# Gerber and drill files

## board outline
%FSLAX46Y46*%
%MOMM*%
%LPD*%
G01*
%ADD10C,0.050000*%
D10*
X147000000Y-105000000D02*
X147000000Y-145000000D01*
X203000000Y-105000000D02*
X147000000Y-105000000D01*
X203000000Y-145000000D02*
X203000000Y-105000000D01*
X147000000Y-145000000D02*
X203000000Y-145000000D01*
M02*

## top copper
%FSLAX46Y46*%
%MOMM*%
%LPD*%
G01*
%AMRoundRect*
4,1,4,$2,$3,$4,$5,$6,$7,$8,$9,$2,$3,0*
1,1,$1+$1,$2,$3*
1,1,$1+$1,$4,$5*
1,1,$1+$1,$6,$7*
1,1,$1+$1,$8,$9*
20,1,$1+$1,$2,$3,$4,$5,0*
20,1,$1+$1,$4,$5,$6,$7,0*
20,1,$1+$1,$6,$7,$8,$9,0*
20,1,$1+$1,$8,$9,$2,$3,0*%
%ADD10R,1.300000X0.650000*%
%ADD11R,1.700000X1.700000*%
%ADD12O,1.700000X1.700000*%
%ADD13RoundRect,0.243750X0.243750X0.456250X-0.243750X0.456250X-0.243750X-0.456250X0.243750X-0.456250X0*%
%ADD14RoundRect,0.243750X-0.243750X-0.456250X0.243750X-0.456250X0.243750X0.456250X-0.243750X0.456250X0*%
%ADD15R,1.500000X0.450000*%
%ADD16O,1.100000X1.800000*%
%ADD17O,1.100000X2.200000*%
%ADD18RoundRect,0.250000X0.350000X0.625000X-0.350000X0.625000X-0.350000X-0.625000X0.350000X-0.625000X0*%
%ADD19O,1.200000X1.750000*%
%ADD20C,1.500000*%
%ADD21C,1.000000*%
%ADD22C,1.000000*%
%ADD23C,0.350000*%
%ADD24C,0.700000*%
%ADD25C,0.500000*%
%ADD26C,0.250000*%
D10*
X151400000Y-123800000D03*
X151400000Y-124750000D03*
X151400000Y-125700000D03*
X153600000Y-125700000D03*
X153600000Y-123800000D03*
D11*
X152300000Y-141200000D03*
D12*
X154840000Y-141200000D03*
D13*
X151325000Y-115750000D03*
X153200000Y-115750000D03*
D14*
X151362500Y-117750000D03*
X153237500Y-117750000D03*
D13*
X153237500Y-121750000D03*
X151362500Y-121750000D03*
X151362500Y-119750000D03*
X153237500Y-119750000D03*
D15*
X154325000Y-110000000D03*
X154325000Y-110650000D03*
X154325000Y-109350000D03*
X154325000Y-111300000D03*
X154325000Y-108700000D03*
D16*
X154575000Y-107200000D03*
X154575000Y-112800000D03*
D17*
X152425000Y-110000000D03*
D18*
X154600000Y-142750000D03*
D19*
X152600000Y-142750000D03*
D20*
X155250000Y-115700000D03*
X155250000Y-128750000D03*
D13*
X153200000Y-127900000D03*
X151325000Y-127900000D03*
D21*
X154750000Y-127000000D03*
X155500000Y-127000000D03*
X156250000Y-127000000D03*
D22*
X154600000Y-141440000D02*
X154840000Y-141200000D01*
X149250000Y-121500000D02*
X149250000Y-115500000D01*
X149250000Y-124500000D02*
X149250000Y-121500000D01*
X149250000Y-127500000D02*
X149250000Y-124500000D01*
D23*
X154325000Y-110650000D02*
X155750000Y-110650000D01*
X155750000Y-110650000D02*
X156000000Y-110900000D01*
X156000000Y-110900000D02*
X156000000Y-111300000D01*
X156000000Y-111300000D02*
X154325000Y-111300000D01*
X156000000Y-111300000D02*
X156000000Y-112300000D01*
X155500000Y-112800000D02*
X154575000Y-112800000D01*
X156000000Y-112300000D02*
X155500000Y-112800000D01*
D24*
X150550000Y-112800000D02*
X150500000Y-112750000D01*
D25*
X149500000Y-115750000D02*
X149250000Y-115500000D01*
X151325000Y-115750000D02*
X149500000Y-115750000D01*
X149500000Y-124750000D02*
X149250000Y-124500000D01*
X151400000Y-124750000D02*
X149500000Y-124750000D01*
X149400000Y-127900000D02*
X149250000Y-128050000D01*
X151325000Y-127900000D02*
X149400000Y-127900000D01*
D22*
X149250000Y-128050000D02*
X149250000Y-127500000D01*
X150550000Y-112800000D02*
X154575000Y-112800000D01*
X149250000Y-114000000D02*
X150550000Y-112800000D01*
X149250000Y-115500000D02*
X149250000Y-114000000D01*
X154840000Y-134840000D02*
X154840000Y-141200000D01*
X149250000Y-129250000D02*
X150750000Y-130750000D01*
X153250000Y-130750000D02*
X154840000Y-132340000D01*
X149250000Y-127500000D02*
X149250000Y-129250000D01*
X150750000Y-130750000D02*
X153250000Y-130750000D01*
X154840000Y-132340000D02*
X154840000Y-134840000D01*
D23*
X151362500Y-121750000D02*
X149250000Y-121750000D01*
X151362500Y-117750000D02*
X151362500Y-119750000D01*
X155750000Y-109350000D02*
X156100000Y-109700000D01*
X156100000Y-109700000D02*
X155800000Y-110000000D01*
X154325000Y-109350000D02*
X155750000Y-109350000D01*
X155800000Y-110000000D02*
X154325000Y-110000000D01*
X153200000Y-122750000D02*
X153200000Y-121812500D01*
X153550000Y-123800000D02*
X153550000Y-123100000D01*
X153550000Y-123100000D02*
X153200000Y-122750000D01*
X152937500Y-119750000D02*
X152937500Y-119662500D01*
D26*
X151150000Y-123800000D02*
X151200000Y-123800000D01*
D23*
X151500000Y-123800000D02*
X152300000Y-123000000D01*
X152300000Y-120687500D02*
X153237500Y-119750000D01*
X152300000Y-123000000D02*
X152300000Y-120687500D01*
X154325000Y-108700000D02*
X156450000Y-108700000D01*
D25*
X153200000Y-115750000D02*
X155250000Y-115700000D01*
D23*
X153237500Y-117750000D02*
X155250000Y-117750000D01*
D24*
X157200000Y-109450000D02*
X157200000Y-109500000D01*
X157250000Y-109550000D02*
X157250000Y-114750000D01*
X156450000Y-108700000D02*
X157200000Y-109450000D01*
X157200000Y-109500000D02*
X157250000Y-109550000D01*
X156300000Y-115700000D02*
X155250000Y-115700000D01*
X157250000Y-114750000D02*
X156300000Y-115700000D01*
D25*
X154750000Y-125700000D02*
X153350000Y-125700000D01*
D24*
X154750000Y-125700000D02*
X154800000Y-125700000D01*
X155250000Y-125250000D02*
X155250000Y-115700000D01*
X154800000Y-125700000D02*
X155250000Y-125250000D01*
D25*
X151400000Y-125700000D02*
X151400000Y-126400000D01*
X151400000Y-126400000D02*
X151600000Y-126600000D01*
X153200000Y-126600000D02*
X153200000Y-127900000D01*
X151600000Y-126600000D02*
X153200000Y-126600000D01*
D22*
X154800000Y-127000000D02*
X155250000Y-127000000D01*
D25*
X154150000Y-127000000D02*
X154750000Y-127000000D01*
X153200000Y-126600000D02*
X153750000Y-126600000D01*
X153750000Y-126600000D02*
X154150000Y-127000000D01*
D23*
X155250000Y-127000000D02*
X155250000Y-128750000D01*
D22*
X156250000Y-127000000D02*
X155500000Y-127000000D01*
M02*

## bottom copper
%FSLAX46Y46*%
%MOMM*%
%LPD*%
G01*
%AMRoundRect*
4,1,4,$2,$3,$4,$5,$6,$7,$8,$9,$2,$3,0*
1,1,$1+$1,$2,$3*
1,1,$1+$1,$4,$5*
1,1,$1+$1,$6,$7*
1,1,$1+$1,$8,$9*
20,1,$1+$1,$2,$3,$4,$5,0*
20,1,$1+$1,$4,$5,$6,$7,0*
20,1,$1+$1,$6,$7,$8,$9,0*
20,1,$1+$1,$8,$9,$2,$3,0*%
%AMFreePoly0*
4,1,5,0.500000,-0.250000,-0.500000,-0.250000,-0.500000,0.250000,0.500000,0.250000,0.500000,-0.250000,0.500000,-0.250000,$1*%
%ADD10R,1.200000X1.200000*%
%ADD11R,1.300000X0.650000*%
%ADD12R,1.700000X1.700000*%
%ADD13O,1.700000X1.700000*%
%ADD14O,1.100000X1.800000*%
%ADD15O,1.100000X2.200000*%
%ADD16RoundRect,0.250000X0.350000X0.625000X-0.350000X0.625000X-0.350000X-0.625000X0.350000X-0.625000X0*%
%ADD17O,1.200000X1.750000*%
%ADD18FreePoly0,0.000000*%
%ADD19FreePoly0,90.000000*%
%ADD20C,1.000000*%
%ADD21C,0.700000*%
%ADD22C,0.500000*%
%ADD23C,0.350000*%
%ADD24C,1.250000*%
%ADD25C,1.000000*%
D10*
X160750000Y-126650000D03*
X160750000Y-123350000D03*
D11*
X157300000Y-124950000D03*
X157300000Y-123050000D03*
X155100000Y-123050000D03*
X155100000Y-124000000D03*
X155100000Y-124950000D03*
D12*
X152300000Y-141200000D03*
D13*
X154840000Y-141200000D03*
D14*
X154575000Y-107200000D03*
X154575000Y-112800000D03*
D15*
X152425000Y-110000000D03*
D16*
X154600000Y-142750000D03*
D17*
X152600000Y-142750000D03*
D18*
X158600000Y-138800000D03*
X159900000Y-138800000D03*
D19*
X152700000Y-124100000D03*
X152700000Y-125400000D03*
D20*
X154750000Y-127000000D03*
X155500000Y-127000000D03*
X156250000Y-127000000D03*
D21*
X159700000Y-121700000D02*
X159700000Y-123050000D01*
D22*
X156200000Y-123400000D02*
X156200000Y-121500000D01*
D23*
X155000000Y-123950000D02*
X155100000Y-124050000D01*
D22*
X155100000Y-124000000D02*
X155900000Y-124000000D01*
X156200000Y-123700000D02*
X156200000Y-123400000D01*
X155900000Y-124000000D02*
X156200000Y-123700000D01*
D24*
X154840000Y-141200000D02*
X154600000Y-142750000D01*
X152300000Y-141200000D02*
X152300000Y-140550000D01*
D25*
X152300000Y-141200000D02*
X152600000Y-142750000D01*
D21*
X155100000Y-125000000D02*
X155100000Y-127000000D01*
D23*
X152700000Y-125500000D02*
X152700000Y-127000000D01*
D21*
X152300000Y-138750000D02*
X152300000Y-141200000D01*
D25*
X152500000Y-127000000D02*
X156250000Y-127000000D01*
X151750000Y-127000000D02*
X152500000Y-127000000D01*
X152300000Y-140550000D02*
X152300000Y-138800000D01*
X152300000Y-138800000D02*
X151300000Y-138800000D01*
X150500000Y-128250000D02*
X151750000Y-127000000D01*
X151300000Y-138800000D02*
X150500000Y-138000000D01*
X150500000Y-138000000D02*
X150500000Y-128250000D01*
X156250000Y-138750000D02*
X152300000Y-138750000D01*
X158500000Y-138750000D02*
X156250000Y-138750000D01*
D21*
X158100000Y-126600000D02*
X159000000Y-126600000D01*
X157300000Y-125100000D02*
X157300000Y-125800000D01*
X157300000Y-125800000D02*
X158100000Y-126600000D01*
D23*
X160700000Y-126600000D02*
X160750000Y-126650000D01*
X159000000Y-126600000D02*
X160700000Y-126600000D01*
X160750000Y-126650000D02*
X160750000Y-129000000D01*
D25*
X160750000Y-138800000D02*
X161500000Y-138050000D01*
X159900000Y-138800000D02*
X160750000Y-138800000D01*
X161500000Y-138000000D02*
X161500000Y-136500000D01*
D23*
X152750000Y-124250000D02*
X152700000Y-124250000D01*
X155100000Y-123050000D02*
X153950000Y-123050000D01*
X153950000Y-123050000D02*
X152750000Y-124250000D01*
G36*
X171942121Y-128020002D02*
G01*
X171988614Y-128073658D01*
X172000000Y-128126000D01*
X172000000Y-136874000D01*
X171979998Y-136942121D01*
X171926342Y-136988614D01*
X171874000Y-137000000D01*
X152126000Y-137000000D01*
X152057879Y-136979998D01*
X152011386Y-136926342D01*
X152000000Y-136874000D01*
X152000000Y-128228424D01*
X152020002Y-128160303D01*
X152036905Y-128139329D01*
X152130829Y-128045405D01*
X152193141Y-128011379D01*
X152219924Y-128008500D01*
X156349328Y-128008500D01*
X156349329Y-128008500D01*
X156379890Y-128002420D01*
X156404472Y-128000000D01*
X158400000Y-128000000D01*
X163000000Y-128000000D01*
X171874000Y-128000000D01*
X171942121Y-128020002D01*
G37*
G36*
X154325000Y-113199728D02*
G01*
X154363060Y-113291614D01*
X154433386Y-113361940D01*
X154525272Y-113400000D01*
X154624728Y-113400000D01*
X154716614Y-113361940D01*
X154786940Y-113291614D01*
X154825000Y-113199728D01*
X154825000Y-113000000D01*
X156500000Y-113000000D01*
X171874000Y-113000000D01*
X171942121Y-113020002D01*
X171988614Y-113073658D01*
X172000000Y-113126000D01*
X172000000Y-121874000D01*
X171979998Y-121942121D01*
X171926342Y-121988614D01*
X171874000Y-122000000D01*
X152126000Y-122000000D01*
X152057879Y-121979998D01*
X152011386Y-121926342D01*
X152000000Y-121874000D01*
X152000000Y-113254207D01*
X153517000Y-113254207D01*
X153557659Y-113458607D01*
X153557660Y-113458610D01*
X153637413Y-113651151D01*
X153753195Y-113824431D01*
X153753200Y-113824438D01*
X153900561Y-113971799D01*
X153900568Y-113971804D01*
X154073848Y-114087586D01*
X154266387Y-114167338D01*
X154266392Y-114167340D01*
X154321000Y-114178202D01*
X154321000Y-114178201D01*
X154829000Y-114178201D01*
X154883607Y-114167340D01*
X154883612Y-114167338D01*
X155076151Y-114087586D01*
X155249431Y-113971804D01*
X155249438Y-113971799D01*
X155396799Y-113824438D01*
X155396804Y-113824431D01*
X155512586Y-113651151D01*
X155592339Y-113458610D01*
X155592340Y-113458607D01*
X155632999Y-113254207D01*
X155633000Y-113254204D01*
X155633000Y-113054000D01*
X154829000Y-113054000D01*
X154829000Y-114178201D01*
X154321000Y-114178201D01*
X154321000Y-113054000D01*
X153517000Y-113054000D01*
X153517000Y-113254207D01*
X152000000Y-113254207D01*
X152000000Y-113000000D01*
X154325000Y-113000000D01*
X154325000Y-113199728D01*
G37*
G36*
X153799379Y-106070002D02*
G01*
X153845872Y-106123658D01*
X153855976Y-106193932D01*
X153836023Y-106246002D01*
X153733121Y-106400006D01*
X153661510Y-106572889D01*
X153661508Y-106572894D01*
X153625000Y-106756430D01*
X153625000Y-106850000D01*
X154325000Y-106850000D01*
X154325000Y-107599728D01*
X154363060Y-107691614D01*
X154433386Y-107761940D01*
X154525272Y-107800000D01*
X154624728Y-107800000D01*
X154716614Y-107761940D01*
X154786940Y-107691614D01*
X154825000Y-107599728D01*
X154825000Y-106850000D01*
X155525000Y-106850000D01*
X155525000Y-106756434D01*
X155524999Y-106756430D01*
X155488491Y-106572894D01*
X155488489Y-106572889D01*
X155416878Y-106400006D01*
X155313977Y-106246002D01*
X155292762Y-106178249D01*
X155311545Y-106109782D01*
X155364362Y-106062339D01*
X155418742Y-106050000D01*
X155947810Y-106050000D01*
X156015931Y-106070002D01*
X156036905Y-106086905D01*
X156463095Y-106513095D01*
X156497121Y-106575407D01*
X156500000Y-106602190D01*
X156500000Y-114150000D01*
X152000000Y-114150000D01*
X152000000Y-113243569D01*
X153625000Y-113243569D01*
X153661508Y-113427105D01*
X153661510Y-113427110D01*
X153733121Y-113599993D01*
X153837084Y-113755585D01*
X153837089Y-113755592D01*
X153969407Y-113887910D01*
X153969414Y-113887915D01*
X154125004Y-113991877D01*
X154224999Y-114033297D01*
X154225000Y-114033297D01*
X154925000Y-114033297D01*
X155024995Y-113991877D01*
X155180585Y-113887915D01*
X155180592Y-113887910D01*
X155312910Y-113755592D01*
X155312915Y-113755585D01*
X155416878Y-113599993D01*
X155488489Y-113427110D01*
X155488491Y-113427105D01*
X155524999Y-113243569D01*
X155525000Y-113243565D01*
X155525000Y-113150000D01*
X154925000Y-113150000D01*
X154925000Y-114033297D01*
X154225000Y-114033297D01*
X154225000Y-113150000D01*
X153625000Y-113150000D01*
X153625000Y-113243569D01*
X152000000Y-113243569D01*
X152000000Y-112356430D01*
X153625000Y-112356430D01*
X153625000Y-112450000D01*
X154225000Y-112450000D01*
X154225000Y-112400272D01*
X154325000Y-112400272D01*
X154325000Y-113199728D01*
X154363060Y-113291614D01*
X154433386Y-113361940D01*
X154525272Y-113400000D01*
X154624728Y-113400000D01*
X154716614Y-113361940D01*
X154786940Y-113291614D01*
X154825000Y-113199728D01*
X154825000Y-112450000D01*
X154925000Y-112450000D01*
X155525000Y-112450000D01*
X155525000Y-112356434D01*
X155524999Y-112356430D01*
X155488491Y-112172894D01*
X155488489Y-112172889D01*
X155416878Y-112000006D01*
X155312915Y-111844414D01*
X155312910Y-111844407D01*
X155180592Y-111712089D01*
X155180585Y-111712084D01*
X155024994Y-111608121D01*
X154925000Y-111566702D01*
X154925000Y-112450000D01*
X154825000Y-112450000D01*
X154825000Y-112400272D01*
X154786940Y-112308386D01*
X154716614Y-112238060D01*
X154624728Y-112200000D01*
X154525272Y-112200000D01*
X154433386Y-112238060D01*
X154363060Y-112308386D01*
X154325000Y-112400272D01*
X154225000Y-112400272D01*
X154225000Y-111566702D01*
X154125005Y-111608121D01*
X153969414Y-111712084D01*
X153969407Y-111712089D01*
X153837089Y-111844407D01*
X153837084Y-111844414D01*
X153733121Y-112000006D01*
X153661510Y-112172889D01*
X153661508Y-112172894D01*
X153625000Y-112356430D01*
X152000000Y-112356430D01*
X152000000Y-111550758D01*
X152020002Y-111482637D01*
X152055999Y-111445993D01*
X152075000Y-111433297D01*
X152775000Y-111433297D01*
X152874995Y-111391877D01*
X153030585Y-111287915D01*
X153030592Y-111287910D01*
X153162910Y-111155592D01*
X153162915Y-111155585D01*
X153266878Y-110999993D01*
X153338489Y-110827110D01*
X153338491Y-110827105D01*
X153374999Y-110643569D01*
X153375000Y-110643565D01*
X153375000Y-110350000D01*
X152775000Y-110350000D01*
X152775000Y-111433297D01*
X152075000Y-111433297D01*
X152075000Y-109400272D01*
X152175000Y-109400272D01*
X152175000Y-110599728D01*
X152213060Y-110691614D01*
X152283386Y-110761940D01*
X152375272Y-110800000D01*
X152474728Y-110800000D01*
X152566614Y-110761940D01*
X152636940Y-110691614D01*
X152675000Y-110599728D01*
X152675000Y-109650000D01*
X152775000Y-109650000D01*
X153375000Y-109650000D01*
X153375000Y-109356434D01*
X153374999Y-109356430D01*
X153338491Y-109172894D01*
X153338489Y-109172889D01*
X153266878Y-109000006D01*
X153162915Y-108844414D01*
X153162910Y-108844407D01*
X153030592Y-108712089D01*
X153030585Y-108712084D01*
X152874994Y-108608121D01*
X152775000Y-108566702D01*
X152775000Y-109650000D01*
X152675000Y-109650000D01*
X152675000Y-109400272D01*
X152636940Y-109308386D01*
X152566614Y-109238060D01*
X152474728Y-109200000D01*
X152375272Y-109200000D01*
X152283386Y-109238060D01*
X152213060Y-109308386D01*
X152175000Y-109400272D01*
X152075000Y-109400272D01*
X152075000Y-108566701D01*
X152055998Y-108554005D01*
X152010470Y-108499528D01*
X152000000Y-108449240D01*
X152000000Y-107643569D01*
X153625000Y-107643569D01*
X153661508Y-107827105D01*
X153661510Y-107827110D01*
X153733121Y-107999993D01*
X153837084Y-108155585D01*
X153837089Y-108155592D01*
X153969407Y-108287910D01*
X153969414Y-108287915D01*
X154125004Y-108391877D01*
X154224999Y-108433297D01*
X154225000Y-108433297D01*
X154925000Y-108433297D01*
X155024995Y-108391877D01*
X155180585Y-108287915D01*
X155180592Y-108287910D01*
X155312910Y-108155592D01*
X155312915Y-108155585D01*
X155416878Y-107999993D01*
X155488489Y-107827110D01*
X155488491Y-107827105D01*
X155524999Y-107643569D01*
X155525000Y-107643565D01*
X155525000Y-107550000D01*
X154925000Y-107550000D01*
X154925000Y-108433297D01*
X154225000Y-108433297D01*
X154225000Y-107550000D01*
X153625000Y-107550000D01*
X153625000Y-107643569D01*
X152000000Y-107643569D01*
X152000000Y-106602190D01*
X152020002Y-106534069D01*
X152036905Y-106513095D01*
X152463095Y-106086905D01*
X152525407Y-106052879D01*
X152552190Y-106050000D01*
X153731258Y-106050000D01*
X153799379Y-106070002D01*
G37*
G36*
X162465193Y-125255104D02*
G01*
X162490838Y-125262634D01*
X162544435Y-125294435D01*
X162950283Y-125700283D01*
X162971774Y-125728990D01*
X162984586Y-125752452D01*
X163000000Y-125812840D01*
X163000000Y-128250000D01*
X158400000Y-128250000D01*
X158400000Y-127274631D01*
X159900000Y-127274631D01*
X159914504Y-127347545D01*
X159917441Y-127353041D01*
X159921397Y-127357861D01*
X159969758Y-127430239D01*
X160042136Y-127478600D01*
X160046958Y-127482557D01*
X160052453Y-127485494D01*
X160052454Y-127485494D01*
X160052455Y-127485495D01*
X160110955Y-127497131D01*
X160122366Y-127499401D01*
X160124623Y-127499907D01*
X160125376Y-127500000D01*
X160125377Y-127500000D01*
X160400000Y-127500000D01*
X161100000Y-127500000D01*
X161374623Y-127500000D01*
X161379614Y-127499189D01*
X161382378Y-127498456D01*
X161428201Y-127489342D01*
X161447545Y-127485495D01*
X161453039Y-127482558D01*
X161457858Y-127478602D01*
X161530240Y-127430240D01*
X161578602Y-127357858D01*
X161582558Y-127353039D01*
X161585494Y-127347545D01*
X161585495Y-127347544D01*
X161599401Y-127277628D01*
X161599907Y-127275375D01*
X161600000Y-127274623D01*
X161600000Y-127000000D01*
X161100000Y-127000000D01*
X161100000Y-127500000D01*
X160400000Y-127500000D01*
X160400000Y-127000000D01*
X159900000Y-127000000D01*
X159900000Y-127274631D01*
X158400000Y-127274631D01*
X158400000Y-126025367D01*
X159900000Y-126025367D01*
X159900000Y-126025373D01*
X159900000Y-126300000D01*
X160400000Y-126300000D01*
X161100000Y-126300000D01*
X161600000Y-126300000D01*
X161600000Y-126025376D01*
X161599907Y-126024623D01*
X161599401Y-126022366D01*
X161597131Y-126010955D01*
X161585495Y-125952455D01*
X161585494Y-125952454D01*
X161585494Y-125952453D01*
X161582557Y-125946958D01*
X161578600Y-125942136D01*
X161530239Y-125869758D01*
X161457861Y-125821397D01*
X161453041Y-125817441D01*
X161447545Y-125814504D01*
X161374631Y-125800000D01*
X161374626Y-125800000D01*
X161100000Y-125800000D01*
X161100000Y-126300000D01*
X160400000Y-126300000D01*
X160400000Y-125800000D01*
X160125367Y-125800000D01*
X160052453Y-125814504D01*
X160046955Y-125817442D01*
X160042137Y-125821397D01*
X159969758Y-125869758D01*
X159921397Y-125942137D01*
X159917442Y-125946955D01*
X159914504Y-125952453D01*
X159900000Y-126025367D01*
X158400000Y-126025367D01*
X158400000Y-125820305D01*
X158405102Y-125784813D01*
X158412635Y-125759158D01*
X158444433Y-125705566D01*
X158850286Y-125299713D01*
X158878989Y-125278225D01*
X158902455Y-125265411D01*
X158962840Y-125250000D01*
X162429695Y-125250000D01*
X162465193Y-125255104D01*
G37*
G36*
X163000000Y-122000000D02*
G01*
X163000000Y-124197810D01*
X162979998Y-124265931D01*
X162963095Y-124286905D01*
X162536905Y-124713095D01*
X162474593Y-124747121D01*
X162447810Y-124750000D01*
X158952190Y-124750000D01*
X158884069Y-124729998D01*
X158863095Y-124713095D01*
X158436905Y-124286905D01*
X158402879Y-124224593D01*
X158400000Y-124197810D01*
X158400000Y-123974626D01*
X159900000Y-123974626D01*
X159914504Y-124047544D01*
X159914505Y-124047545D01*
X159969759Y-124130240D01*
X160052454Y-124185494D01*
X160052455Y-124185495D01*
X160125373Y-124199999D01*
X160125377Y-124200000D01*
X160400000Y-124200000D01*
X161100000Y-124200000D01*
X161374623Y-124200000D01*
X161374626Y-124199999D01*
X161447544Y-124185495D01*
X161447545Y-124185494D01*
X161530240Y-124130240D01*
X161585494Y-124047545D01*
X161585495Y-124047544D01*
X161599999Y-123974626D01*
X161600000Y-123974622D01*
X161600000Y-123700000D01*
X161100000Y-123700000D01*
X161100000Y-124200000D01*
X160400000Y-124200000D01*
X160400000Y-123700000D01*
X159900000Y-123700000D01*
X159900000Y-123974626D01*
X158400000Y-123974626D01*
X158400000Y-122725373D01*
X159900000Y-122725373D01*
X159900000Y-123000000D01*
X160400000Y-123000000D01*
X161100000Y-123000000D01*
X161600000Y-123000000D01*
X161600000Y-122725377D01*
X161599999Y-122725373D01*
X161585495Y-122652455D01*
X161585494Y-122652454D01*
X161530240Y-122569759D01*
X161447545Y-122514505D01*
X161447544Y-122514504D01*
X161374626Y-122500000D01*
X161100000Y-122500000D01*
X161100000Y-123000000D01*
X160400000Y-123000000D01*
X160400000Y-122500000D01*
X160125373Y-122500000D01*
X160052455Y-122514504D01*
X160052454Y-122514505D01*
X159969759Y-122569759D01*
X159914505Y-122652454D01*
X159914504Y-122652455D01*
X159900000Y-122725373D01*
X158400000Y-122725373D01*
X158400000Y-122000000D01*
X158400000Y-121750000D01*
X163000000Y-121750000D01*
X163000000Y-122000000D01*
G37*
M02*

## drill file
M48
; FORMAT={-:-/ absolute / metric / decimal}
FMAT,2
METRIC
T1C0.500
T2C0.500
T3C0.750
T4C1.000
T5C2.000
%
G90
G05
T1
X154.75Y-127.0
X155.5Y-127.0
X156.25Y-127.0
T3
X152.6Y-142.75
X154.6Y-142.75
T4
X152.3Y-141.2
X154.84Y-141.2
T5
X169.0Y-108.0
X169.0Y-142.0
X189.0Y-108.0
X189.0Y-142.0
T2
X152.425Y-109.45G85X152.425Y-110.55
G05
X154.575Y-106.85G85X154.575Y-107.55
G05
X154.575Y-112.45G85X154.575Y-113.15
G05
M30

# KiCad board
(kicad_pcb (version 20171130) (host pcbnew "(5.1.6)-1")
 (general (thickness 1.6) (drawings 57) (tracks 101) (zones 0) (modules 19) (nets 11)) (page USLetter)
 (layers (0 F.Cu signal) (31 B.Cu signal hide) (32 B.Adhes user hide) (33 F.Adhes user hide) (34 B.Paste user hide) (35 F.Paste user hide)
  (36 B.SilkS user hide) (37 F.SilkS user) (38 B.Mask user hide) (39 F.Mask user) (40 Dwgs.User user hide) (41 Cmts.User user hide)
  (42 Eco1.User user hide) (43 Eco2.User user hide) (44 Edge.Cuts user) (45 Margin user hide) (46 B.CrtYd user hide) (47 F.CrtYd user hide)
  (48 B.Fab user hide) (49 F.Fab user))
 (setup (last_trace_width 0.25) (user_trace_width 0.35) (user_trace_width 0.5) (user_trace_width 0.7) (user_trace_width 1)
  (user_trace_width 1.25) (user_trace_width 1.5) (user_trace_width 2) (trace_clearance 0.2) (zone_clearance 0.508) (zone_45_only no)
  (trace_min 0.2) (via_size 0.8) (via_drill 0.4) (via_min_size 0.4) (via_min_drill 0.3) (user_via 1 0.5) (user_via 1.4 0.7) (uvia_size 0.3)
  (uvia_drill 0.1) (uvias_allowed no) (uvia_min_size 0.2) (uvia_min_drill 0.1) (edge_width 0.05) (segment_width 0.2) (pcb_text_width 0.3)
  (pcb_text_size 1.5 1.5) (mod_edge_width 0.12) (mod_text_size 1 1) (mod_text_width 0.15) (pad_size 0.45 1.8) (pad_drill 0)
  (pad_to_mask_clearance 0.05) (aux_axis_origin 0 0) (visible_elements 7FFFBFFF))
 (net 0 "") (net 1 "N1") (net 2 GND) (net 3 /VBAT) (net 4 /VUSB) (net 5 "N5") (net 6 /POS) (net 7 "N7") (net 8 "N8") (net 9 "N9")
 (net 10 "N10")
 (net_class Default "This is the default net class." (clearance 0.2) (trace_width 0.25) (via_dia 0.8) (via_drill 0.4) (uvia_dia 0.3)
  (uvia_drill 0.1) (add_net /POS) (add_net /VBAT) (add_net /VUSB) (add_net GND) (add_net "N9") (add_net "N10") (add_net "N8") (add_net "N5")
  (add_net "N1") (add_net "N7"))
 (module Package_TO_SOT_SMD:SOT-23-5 (layer F.Cu) (at 152.5 124.75)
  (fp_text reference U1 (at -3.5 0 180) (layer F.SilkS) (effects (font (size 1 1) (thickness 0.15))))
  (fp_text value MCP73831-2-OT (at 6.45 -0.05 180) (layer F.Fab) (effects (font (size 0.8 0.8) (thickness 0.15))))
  (pad 1 smd rect (at -1.1 -0.95) (size 1.3 0.65) (layers F.Cu F.Paste F.Mask) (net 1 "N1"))
  (pad 2 smd rect (at -1.1 0) (size 1.3 0.65) (layers F.Cu F.Paste F.Mask) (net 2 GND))
  (pad 3 smd rect (at -1.1 0.95) (size 1.3 0.65) (layers F.Cu F.Paste F.Mask) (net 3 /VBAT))
  (pad 4 smd rect (at 1.1 0.95) (size 1.3 0.65) (layers F.Cu F.Paste F.Mask) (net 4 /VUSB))
  (pad 5 smd rect (at 1.1 -0.95) (size 1.3 0.65) (layers F.Cu F.Paste F.Mask) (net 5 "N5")))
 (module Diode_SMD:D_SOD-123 (layer B.Cu) (at 160.75 125 90)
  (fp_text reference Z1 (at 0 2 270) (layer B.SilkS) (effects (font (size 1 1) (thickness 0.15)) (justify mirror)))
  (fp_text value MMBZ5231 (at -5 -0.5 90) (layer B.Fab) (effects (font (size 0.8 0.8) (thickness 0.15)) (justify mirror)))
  (pad 1 smd rect (at -1.65 0 90) (size 1.2 1.2) (layers B.Cu B.Paste B.Mask) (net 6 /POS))
  (pad 2 smd rect (at 1.65 0 90) (size 1.2 1.2) (layers B.Cu B.Paste B.Mask) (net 2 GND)))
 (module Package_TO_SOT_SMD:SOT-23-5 (layer B.Cu) (at 156.2 124)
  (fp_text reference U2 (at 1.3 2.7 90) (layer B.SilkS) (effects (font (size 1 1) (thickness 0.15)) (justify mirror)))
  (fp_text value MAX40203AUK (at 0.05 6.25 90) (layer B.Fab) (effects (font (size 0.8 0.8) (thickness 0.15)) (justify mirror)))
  (pad 5 smd rect (at 1.1 0.95) (size 1.3 0.65) (layers B.Cu B.Paste B.Mask) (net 6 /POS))
  (pad 4 smd rect (at 1.1 -0.95) (size 1.3 0.65) (layers B.Cu B.Paste B.Mask) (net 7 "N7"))
  (pad 3 smd rect (at -1.1 -0.95) (size 1.3 0.65) (layers B.Cu B.Paste B.Mask) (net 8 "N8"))
  (pad 2 smd rect (at -1.1 0) (size 1.3 0.65) (layers B.Cu B.Paste B.Mask) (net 2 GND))
  (pad 1 smd rect (at -1.1 0.95) (size 1.3 0.65) (layers B.Cu B.Paste B.Mask) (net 3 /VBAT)))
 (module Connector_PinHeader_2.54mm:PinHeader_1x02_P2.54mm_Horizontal (layer F.Cu) (at 152.3 141.2 90)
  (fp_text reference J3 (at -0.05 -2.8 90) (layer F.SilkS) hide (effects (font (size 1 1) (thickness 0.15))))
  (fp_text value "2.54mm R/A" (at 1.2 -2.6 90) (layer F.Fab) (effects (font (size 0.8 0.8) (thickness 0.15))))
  (pad 1 thru_hole rect (at 0 0 90) (size 1.7 1.7) (drill 1) (layers *.Cu *.Mask) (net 3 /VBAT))
  (pad 2 thru_hole oval (at 0 2.54 90) (size 1.7 1.7) (drill 1) (layers *.Cu *.Mask) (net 2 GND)))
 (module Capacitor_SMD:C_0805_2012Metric (layer F.Cu) (at 152.2625 115.75 180)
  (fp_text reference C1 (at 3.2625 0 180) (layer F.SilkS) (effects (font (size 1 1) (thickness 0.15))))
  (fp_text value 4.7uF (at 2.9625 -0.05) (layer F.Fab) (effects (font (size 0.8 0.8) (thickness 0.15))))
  (pad 2 smd roundrect (at 0.9375 0 180) (size 0.975 1.4) (layers F.Cu F.Paste F.Mask) (roundrect_rratio 0.25) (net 2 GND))
  (pad 1 smd roundrect (at -0.9375 0 180) (size 0.975 1.4) (layers F.Cu F.Paste F.Mask) (roundrect_rratio 0.25) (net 4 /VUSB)))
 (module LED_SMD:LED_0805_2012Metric (layer F.Cu) (at 152.3 117.75)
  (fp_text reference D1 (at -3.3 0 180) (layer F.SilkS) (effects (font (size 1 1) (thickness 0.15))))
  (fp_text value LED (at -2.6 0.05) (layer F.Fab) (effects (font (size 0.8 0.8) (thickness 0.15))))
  (pad 1 smd roundrect (at -0.9375 0) (size 0.975 1.4) (layers F.Cu F.Paste F.Mask) (roundrect_rratio 0.25) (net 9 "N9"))
  (pad 2 smd roundrect (at 0.9375 0) (size 0.975 1.4) (layers F.Cu F.Paste F.Mask) (roundrect_rratio 0.25) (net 4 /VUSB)))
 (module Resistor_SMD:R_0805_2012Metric (layer F.Cu) (at 152.3 121.75 180)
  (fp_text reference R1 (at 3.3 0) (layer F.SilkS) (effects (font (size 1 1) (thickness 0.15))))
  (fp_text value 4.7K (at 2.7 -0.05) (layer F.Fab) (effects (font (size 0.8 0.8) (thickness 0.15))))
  (pad 1 smd roundrect (at -0.9375 0 180) (size 0.975 1.4) (layers F.Cu F.Paste F.Mask) (roundrect_rratio 0.25) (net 5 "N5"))
  (pad 2 smd roundrect (at 0.9375 0 180) (size 0.975 1.4) (layers F.Cu F.Paste F.Mask) (roundrect_rratio 0.25) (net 2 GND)))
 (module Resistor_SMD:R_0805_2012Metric (layer F.Cu) (at 152.3 119.75 180)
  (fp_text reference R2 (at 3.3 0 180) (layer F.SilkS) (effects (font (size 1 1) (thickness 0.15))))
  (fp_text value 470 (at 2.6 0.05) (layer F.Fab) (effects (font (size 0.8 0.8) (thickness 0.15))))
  (pad 2 smd roundrect (at 0.9375 0 180) (size 0.975 1.4) (layers F.Cu F.Paste F.Mask) (roundrect_rratio 0.25) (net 9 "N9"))
  (pad 1 smd roundrect (at -0.9375 0 180) (size 0.975 1.4) (layers F.Cu F.Paste F.Mask) (roundrect_rratio 0.25) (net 1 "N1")))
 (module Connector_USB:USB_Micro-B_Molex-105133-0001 (layer F.Cu) (at 153.5 110 270)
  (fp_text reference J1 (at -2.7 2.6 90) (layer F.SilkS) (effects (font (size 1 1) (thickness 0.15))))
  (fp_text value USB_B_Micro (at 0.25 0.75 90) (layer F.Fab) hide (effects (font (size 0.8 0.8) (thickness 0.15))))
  (pad 3 smd rect (at 0 -0.825 270) (size 0.45 1.5) (layers F.Cu F.Paste F.Mask) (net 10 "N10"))
  (pad 4 smd rect (at 0.65 -0.825 270) (size 0.45 1.5) (layers F.Cu F.Paste F.Mask) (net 2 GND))
  (pad 2 smd rect (at -0.65 -0.825 270) (size 0.45 1.5) (layers F.Cu F.Paste F.Mask) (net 10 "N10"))
  (pad 5 smd rect (at 1.3 -0.825 270) (size 0.45 1.5) (layers F.Cu F.Paste F.Mask) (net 2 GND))
  (pad 1 smd rect (at -1.3 -0.825 270) (size 0.45 1.5) (layers F.Cu F.Paste F.Mask) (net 4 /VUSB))
  (pad 6 thru_hole oval (at -2.8 -1.075 270) (size 1.8 1.1) (drill oval 1.2 0.5) (layers *.Cu *.Mask) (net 2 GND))
  (pad 6 thru_hole oval (at 2.8 -1.075 270) (size 1.8 1.1) (drill oval 1.2 0.5) (layers *.Cu *.Mask) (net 2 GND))
  (pad 6 thru_hole oval (at 0 1.075 270) (size 2.2 1.1) (drill oval 1.6 0.5) (layers *.Cu *.Mask) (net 2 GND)))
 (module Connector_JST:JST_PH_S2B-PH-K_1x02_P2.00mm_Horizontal (layer F.Cu) (at 154.6 142.75 180)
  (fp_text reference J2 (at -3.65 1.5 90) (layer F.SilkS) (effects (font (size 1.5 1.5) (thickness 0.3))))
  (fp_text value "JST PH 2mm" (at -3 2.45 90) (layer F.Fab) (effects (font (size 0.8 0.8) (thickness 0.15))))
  (pad 1 thru_hole roundrect (at 0 0 180) (size 1.2 1.75) (drill 0.75) (layers *.Cu *.Mask) (roundrect_rratio 0.208333) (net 2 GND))
  (pad 2 thru_hole oval (at 2 0 180) (size 1.2 1.75) (drill 0.75) (layers *.Cu *.Mask) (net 3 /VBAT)))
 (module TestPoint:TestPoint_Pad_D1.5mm (layer F.Cu) (at 155.25 115.7 270)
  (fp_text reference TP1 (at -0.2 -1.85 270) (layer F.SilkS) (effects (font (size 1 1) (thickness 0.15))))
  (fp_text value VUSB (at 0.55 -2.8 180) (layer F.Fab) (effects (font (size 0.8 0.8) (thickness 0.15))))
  (pad 1 smd circle (at 0 0 270) (size 1.5 1.5) (layers F.Cu F.Mask) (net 4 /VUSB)))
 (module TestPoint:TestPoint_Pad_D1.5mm (layer F.Cu) (at 155.25 128.75)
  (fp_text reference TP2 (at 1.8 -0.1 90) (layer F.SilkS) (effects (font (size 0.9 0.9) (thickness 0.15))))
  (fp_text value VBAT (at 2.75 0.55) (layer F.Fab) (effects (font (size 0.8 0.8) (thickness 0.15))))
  (pad 1 smd circle (at 0 0) (size 1.5 1.5) (layers F.Cu F.Mask) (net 3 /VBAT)))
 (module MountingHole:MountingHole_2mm (layer F.Cu) (at 189 108)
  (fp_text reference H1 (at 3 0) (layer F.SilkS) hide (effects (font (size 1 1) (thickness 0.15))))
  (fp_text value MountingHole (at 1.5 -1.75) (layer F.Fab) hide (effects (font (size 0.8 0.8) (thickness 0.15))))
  (pad "" np_thru_hole circle (at 0 0) (size 2 2) (drill 2) (layers *.Cu *.Mask)))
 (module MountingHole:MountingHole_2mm (layer F.Cu) (at 169 108)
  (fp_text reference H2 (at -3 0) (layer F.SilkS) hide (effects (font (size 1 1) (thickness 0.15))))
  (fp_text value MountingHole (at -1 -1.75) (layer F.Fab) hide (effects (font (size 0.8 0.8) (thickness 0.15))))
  (pad "" np_thru_hole circle (at 0 0) (size 2 2) (drill 2) (layers *.Cu *.Mask)))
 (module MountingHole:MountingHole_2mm (layer F.Cu) (at 189 142)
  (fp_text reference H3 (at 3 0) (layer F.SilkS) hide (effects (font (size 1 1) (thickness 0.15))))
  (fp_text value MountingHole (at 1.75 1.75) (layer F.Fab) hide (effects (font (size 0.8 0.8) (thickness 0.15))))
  (pad "" np_thru_hole circle (at 0 0) (size 2 2) (drill 2) (layers *.Cu *.Mask)))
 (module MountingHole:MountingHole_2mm (layer F.Cu) (at 169 142)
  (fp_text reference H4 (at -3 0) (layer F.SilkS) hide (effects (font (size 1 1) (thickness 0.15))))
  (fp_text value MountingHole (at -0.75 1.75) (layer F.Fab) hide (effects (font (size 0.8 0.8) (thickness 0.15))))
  (pad "" np_thru_hole circle (at 0 0) (size 2 2) (drill 2) (layers *.Cu *.Mask)))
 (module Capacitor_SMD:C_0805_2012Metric (layer F.Cu) (at 152.2625 127.9 180)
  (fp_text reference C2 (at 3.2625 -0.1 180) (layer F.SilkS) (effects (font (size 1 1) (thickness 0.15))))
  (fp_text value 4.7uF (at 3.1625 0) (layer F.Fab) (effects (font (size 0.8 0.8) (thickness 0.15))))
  (pad 1 smd roundrect (at -0.9375 0 180) (size 0.975 1.4) (layers F.Cu F.Paste F.Mask) (roundrect_rratio 0.25) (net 3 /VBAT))
  (pad 2 smd roundrect (at 0.9375 0 180) (size 0.975 1.4) (layers F.Cu F.Paste F.Mask) (roundrect_rratio 0.25) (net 2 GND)))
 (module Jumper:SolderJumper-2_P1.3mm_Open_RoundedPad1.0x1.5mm (layer B.Cu) (at 159.25 138.8)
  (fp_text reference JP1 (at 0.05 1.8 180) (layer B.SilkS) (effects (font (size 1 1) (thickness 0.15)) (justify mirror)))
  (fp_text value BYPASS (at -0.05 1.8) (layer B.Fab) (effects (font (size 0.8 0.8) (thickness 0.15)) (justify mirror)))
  (pad 1 smd custom (at -0.65 0) (size 1 0.5) (layers B.Cu B.Mask) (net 3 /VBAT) (zone_connect 2)
   (options (clearance outline) (anchor rect)) (primitives))
  (pad 2 smd custom (at 0.65 0) (size 1 0.5) (layers B.Cu B.Mask) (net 6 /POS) (zone_connect 2) (options (clearance outline) (anchor rect))
   (primitives)))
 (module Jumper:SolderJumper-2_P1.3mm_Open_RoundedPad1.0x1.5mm (layer B.Cu) (at 152.7 124.75 90)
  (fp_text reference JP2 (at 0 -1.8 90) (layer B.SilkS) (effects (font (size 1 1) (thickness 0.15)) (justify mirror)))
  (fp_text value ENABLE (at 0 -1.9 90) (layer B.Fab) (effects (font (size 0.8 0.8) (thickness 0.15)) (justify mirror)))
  (pad 2 smd custom (at 0.65 0 90) (size 1 0.5) (layers B.Cu B.Mask) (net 8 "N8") (zone_connect 2)
   (options (clearance outline) (anchor rect)) (primitives))
  (pad 1 smd custom (at -0.65 0 90) (size 1 0.5) (layers B.Cu B.Mask) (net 3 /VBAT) (zone_connect 2)
   (options (clearance outline) (anchor rect)) (primitives)))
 (gr_line (start 147 105) (end 147 145) (layer Edge.Cuts) (width 0.05))
 (gr_line (start 203 105) (end 147 105) (layer Edge.Cuts) (width 0.05))
 (gr_line (start 203 145) (end 203 105) (layer Edge.Cuts) (width 0.05))
 (gr_line (start 147 145) (end 203 145) (layer Edge.Cuts) (width 0.05))
 (segment (start 159.7 121.7) (end 159.7 123.05) (width 0.7) (layer B.Cu) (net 2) (status 20))
 (segment (start 156.2 123.4) (end 156.2 121.5) (width 0.5) (layer B.Cu) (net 2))
 (segment (start 155 123.95) (end 155.1 124.05) (width 0.35) (layer B.Cu) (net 2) (status 30))
 (segment (start 155.1 124) (end 155.9 124) (width 0.5) (layer B.Cu) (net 2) (status 10))
 (segment (start 156.2 123.7) (end 156.2 123.4) (width 0.5) (layer B.Cu) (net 2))
 (segment (start 155.9 124) (end 156.2 123.7) (width 0.5) (layer B.Cu) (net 2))
 (segment (start 154.6 141.44) (end 154.84 141.2) (width 1) (layer F.Cu) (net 2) (status 30))
 (segment (start 149.25 121.5) (end 149.25 115.5) (width 1) (layer F.Cu) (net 2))
 (segment (start 149.25 124.5) (end 149.25 121.5) (width 1) (layer F.Cu) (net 2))
 (segment (start 149.25 127.5) (end 149.25 124.5) (width 1) (layer F.Cu) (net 2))
 (segment (start 154.325 110.65) (end 155.75 110.65) (width 0.35) (layer F.Cu) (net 2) (status 10))
 (segment (start 155.75 110.65) (end 156 110.9) (width 0.35) (layer F.Cu) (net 2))
 (segment (start 156 110.9) (end 156 111.3) (width 0.35) (layer F.Cu) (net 2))
 (segment (start 156 111.3) (end 154.325 111.3) (width 0.35) (layer F.Cu) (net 2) (status 20))
 (segment (start 156 111.3) (end 156 112.3) (width 0.35) (layer F.Cu) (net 2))
 (segment (start 155.5 112.8) (end 154.575 112.8) (width 0.35) (layer F.Cu) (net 2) (status 20))
 (segment (start 156 112.3) (end 155.5 112.8) (width 0.35) (layer F.Cu) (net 2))
 (segment (start 150.55 112.8) (end 150.5 112.75) (width 0.7) (layer F.Cu) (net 2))
 (segment (start 149.5 115.75) (end 149.25 115.5) (width 0.5) (layer F.Cu) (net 2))
 (segment (start 151.325 115.75) (end 149.5 115.75) (width 0.5) (layer F.Cu) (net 2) (status 10))
 (segment (start 149.5 124.75) (end 149.25 124.5) (width 0.5) (layer F.Cu) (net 2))
 (segment (start 151.4 124.75) (end 149.5 124.75) (width 0.5) (layer F.Cu) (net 2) (status 10))
 (segment (start 149.4 127.9) (end 149.25 128.05) (width 0.5) (layer F.Cu) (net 2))
 (segment (start 151.325 127.9) (end 149.4 127.9) (width 0.5) (layer F.Cu) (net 2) (status 10))
 (segment (start 149.25 128.05) (end 149.25 127.5) (width 1) (layer F.Cu) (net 2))
 (segment (start 154.84 141.2) (end 154.6 142.75) (width 1.25) (layer B.Cu) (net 2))
 (segment (start 150.55 112.8) (end 154.575 112.8) (width 1) (layer F.Cu) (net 2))
 (segment (start 149.25 114) (end 150.55 112.8) (width 1) (layer F.Cu) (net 2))
 (segment (start 149.25 115.5) (end 149.25 114) (width 1) (layer F.Cu) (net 2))
 (segment (start 154.84 134.84) (end 154.84 141.2) (width 1) (layer F.Cu) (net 2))
 (segment (start 149.25 129.25) (end 150.75 130.75) (width 1) (layer F.Cu) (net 2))
 (segment (start 153.25 130.75) (end 154.84 132.34) (width 1) (layer F.Cu) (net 2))
 (segment (start 149.25 127.5) (end 149.25 129.25) (width 1) (layer F.Cu) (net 2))
 (segment (start 150.75 130.75) (end 153.25 130.75) (width 1) (layer F.Cu) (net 2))
 (segment (start 154.84 132.34) (end 154.84 134.84) (width 1) (layer F.Cu) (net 2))
 (segment (start 151.3625 121.75) (end 149.25 121.75) (width 0.35) (layer F.Cu) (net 2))
 (segment (start 151.3625 117.75) (end 151.3625 119.75) (width 0.35) (layer F.Cu) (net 9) (status 30))
 (segment (start 155.75 109.35) (end 156.1 109.7) (width 0.35) (layer F.Cu) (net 10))
 (segment (start 156.1 109.7) (end 155.8 110) (width 0.35) (layer F.Cu) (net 10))
 (segment (start 154.325 109.35) (end 155.75 109.35) (width 0.35) (layer F.Cu) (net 10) (status 10))
 (segment (start 155.8 110) (end 154.325 110) (width 0.35) (layer F.Cu) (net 10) (status 20))
 (segment (start 153.2 122.75) (end 153.2 121.8125) (width 0.35) (layer F.Cu) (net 5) (status 20))
 (segment (start 153.55 123.8) (end 153.55 123.1) (width 0.35) (layer F.Cu) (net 5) (status 10))
 (segment (start 153.55 123.1) (end 153.2 122.75) (width 0.35) (layer F.Cu) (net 5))
 (segment (start 152.9375 119.75) (end 152.9375 119.6625) (width 0.35) (layer F.Cu) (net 1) (status 30))
 (segment (start 151.15 123.8) (end 151.2 123.8) (width 0.25) (layer F.Cu) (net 1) (status 30))
 (segment (start 151.5 123.8) (end 152.3 123) (width 0.35) (layer F.Cu) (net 1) (status 10))
 (segment (start 152.3 120.6875) (end 153.2375 119.75) (width 0.35) (layer F.Cu) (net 1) (status 20))
 (segment (start 152.3 123) (end 152.3 120.6875) (width 0.35) (layer F.Cu) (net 1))
 (segment (start 154.325 108.7) (end 156.45 108.7) (width 0.35) (layer F.Cu) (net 4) (status 10))
 (segment (start 153.2 115.75) (end 155.25 115.7) (width 0.5) (layer F.Cu) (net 4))
 (segment (start 153.2375 117.75) (end 155.25 117.75) (width 0.35) (layer F.Cu) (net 4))
 (segment (start 157.2 109.45) (end 157.2 109.5) (width 0.7) (layer F.Cu) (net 4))
 (segment (start 157.25 109.55) (end 157.25 114.75) (width 0.7) (layer F.Cu) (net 4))
 (segment (start 156.45 108.7) (end 157.2 109.45) (width 0.7) (layer F.Cu) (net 4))
 (segment (start 157.2 109.5) (end 157.25 109.55) (width 0.7) (layer F.Cu) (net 4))
 (segment (start 156.3 115.7) (end 155.25 115.7) (width 0.7) (layer F.Cu) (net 4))
 (segment (start 157.25 114.75) (end 156.3 115.7) (width 0.7) (layer F.Cu) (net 4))
 (segment (start 154.75 125.7) (end 153.35 125.7) (width 0.5) (layer F.Cu) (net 4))
 (segment (start 154.75 125.7) (end 154.8 125.7) (width 0.7) (layer F.Cu) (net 4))
 (segment (start 155.25 125.25) (end 155.25 115.7) (width 0.7) (layer F.Cu) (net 4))
 (segment (start 154.8 125.7) (end 155.25 125.25) (width 0.7) (layer F.Cu) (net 4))
 (segment (start 151.4 125.7) (end 151.4 126.4) (width 0.5) (layer F.Cu) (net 3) (status 10))
 (segment (start 151.4 126.4) (end 151.6 126.6) (width 0.5) (layer F.Cu) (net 3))
 (segment (start 153.2 126.6) (end 153.2 127.9) (width 0.5) (layer F.Cu) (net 3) (status 20))
 (segment (start 151.6 126.6) (end 153.2 126.6) (width 0.5) (layer F.Cu) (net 3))
 (via (at 154.75 127) (size 1) (drill 0.5) (layers F.Cu B.Cu) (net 3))
 (via (at 155.5 127) (size 1) (drill 0.5) (layers F.Cu B.Cu) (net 3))
 (segment (start 152.3 141.2) (end 152.3 140.55) (width 1.25) (layer B.Cu) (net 3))
 (segment (start 152.3 141.2) (end 152.6 142.75) (width 1) (layer B.Cu) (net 3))
 (segment (start 154.8 127) (end 155.25 127) (width 1) (layer F.Cu) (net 3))
 (segment (start 155.1 125) (end 155.1 127) (width 0.7) (layer B.Cu) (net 3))
 (segment (start 154.15 127) (end 154.75 127) (width 0.5) (layer F.Cu) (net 3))
 (segment (start 153.2 126.6) (end 153.75 126.6) (width 0.5) (layer F.Cu) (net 3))
 (segment (start 153.75 126.6) (end 154.15 127) (width 0.5) (layer F.Cu) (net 3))
 (segment (start 155.25 127) (end 155.25 128.75) (width 0.35) (layer F.Cu) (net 3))
 (segment (start 152.7 125.5) (end 152.7 127) (width 0.35) (layer B.Cu) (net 3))
 (segment (start 152.3 138.75) (end 152.3 141.2) (width 0.7) (layer B.Cu) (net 3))
 (via (at 156.25 127) (size 1) (drill 0.5) (layers F.Cu B.Cu) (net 3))
 (segment (start 156.25 127) (end 155.5 127) (width 1) (layer F.Cu) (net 3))
 (segment (start 152.5 127) (end 156.25 127) (width 1) (layer B.Cu) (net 3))
 (segment (start 151.75 127) (end 152.5 127) (width 1) (layer B.Cu) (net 3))
 (segment (start 152.3 140.55) (end 152.3 138.8) (width 1) (layer B.Cu) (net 3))
 (segment (start 152.3 138.8) (end 151.3 138.8) (width 1) (layer B.Cu) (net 3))
 (segment (start 150.5 128.25) (end 151.75 127) (width 1) (layer B.Cu) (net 3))
 (segment (start 151.3 138.8) (end 150.5 138) (width 1) (layer B.Cu) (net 3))
 (segment (start 150.5 138) (end 150.5 128.25) (width 1) (layer B.Cu) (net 3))
 (segment (start 156.25 138.75) (end 152.3 138.75) (width 1) (layer B.Cu) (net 3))
 (segment (start 158.5 138.75) (end 156.25 138.75) (width 1) (layer B.Cu) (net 3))
 (segment (start 158.1 126.6) (end 159 126.6) (width 0.7) (layer B.Cu) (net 6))
 (segment (start 157.3 125.1) (end 157.3 125.8) (width 0.7) (layer B.Cu) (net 6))
 (segment (start 157.3 125.8) (end 158.1 126.6) (width 0.7) (layer B.Cu) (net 6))
 (segment (start 160.7 126.6) (end 160.75 126.65) (width 0.35) (layer B.Cu) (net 6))
 (segment (start 159 126.6) (end 160.7 126.6) (width 0.35) (layer B.Cu) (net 6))
 (segment (start 160.75 126.65) (end 160.75 129) (width 0.35) (layer B.Cu) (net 6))
 (segment (start 160.75 138.8) (end 161.5 138.05) (width 1) (layer B.Cu) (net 6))
 (segment (start 159.9 138.8) (end 160.75 138.8) (width 1) (layer B.Cu) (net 6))
 (segment (start 161.5 138) (end 161.5 136.5) (width 1) (layer B.Cu) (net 6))
 (segment (start 152.75 124.25) (end 152.7 124.25) (width 0.35) (layer B.Cu) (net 8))
 (segment (start 155.1 123.05) (end 153.95 123.05) (width 0.35) (layer B.Cu) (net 8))
 (segment (start 153.95 123.05) (end 152.75 124.25) (width 0.35) (layer B.Cu) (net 8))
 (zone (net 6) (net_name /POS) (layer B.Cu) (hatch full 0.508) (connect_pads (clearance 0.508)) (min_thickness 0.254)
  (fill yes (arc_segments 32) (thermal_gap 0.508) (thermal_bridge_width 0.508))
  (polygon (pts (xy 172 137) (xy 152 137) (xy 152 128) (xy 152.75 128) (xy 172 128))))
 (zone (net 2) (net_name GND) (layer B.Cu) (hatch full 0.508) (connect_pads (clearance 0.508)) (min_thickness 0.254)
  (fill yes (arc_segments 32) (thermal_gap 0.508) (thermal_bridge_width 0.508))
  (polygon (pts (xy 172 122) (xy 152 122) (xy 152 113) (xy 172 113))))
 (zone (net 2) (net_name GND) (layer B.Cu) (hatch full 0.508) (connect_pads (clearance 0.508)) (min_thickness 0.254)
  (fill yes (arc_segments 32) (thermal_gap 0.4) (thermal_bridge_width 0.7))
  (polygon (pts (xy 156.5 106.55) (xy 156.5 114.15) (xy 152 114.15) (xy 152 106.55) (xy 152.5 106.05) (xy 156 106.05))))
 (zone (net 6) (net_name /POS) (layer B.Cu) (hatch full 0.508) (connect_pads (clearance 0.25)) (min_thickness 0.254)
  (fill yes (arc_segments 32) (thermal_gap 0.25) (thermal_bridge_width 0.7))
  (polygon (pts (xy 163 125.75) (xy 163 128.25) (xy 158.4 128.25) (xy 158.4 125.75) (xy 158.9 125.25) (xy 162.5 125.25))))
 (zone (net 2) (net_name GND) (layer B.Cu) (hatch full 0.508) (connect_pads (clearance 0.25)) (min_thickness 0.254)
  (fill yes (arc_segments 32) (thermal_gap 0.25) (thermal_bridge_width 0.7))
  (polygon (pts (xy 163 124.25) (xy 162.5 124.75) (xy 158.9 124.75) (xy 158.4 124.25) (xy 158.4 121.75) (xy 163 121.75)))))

